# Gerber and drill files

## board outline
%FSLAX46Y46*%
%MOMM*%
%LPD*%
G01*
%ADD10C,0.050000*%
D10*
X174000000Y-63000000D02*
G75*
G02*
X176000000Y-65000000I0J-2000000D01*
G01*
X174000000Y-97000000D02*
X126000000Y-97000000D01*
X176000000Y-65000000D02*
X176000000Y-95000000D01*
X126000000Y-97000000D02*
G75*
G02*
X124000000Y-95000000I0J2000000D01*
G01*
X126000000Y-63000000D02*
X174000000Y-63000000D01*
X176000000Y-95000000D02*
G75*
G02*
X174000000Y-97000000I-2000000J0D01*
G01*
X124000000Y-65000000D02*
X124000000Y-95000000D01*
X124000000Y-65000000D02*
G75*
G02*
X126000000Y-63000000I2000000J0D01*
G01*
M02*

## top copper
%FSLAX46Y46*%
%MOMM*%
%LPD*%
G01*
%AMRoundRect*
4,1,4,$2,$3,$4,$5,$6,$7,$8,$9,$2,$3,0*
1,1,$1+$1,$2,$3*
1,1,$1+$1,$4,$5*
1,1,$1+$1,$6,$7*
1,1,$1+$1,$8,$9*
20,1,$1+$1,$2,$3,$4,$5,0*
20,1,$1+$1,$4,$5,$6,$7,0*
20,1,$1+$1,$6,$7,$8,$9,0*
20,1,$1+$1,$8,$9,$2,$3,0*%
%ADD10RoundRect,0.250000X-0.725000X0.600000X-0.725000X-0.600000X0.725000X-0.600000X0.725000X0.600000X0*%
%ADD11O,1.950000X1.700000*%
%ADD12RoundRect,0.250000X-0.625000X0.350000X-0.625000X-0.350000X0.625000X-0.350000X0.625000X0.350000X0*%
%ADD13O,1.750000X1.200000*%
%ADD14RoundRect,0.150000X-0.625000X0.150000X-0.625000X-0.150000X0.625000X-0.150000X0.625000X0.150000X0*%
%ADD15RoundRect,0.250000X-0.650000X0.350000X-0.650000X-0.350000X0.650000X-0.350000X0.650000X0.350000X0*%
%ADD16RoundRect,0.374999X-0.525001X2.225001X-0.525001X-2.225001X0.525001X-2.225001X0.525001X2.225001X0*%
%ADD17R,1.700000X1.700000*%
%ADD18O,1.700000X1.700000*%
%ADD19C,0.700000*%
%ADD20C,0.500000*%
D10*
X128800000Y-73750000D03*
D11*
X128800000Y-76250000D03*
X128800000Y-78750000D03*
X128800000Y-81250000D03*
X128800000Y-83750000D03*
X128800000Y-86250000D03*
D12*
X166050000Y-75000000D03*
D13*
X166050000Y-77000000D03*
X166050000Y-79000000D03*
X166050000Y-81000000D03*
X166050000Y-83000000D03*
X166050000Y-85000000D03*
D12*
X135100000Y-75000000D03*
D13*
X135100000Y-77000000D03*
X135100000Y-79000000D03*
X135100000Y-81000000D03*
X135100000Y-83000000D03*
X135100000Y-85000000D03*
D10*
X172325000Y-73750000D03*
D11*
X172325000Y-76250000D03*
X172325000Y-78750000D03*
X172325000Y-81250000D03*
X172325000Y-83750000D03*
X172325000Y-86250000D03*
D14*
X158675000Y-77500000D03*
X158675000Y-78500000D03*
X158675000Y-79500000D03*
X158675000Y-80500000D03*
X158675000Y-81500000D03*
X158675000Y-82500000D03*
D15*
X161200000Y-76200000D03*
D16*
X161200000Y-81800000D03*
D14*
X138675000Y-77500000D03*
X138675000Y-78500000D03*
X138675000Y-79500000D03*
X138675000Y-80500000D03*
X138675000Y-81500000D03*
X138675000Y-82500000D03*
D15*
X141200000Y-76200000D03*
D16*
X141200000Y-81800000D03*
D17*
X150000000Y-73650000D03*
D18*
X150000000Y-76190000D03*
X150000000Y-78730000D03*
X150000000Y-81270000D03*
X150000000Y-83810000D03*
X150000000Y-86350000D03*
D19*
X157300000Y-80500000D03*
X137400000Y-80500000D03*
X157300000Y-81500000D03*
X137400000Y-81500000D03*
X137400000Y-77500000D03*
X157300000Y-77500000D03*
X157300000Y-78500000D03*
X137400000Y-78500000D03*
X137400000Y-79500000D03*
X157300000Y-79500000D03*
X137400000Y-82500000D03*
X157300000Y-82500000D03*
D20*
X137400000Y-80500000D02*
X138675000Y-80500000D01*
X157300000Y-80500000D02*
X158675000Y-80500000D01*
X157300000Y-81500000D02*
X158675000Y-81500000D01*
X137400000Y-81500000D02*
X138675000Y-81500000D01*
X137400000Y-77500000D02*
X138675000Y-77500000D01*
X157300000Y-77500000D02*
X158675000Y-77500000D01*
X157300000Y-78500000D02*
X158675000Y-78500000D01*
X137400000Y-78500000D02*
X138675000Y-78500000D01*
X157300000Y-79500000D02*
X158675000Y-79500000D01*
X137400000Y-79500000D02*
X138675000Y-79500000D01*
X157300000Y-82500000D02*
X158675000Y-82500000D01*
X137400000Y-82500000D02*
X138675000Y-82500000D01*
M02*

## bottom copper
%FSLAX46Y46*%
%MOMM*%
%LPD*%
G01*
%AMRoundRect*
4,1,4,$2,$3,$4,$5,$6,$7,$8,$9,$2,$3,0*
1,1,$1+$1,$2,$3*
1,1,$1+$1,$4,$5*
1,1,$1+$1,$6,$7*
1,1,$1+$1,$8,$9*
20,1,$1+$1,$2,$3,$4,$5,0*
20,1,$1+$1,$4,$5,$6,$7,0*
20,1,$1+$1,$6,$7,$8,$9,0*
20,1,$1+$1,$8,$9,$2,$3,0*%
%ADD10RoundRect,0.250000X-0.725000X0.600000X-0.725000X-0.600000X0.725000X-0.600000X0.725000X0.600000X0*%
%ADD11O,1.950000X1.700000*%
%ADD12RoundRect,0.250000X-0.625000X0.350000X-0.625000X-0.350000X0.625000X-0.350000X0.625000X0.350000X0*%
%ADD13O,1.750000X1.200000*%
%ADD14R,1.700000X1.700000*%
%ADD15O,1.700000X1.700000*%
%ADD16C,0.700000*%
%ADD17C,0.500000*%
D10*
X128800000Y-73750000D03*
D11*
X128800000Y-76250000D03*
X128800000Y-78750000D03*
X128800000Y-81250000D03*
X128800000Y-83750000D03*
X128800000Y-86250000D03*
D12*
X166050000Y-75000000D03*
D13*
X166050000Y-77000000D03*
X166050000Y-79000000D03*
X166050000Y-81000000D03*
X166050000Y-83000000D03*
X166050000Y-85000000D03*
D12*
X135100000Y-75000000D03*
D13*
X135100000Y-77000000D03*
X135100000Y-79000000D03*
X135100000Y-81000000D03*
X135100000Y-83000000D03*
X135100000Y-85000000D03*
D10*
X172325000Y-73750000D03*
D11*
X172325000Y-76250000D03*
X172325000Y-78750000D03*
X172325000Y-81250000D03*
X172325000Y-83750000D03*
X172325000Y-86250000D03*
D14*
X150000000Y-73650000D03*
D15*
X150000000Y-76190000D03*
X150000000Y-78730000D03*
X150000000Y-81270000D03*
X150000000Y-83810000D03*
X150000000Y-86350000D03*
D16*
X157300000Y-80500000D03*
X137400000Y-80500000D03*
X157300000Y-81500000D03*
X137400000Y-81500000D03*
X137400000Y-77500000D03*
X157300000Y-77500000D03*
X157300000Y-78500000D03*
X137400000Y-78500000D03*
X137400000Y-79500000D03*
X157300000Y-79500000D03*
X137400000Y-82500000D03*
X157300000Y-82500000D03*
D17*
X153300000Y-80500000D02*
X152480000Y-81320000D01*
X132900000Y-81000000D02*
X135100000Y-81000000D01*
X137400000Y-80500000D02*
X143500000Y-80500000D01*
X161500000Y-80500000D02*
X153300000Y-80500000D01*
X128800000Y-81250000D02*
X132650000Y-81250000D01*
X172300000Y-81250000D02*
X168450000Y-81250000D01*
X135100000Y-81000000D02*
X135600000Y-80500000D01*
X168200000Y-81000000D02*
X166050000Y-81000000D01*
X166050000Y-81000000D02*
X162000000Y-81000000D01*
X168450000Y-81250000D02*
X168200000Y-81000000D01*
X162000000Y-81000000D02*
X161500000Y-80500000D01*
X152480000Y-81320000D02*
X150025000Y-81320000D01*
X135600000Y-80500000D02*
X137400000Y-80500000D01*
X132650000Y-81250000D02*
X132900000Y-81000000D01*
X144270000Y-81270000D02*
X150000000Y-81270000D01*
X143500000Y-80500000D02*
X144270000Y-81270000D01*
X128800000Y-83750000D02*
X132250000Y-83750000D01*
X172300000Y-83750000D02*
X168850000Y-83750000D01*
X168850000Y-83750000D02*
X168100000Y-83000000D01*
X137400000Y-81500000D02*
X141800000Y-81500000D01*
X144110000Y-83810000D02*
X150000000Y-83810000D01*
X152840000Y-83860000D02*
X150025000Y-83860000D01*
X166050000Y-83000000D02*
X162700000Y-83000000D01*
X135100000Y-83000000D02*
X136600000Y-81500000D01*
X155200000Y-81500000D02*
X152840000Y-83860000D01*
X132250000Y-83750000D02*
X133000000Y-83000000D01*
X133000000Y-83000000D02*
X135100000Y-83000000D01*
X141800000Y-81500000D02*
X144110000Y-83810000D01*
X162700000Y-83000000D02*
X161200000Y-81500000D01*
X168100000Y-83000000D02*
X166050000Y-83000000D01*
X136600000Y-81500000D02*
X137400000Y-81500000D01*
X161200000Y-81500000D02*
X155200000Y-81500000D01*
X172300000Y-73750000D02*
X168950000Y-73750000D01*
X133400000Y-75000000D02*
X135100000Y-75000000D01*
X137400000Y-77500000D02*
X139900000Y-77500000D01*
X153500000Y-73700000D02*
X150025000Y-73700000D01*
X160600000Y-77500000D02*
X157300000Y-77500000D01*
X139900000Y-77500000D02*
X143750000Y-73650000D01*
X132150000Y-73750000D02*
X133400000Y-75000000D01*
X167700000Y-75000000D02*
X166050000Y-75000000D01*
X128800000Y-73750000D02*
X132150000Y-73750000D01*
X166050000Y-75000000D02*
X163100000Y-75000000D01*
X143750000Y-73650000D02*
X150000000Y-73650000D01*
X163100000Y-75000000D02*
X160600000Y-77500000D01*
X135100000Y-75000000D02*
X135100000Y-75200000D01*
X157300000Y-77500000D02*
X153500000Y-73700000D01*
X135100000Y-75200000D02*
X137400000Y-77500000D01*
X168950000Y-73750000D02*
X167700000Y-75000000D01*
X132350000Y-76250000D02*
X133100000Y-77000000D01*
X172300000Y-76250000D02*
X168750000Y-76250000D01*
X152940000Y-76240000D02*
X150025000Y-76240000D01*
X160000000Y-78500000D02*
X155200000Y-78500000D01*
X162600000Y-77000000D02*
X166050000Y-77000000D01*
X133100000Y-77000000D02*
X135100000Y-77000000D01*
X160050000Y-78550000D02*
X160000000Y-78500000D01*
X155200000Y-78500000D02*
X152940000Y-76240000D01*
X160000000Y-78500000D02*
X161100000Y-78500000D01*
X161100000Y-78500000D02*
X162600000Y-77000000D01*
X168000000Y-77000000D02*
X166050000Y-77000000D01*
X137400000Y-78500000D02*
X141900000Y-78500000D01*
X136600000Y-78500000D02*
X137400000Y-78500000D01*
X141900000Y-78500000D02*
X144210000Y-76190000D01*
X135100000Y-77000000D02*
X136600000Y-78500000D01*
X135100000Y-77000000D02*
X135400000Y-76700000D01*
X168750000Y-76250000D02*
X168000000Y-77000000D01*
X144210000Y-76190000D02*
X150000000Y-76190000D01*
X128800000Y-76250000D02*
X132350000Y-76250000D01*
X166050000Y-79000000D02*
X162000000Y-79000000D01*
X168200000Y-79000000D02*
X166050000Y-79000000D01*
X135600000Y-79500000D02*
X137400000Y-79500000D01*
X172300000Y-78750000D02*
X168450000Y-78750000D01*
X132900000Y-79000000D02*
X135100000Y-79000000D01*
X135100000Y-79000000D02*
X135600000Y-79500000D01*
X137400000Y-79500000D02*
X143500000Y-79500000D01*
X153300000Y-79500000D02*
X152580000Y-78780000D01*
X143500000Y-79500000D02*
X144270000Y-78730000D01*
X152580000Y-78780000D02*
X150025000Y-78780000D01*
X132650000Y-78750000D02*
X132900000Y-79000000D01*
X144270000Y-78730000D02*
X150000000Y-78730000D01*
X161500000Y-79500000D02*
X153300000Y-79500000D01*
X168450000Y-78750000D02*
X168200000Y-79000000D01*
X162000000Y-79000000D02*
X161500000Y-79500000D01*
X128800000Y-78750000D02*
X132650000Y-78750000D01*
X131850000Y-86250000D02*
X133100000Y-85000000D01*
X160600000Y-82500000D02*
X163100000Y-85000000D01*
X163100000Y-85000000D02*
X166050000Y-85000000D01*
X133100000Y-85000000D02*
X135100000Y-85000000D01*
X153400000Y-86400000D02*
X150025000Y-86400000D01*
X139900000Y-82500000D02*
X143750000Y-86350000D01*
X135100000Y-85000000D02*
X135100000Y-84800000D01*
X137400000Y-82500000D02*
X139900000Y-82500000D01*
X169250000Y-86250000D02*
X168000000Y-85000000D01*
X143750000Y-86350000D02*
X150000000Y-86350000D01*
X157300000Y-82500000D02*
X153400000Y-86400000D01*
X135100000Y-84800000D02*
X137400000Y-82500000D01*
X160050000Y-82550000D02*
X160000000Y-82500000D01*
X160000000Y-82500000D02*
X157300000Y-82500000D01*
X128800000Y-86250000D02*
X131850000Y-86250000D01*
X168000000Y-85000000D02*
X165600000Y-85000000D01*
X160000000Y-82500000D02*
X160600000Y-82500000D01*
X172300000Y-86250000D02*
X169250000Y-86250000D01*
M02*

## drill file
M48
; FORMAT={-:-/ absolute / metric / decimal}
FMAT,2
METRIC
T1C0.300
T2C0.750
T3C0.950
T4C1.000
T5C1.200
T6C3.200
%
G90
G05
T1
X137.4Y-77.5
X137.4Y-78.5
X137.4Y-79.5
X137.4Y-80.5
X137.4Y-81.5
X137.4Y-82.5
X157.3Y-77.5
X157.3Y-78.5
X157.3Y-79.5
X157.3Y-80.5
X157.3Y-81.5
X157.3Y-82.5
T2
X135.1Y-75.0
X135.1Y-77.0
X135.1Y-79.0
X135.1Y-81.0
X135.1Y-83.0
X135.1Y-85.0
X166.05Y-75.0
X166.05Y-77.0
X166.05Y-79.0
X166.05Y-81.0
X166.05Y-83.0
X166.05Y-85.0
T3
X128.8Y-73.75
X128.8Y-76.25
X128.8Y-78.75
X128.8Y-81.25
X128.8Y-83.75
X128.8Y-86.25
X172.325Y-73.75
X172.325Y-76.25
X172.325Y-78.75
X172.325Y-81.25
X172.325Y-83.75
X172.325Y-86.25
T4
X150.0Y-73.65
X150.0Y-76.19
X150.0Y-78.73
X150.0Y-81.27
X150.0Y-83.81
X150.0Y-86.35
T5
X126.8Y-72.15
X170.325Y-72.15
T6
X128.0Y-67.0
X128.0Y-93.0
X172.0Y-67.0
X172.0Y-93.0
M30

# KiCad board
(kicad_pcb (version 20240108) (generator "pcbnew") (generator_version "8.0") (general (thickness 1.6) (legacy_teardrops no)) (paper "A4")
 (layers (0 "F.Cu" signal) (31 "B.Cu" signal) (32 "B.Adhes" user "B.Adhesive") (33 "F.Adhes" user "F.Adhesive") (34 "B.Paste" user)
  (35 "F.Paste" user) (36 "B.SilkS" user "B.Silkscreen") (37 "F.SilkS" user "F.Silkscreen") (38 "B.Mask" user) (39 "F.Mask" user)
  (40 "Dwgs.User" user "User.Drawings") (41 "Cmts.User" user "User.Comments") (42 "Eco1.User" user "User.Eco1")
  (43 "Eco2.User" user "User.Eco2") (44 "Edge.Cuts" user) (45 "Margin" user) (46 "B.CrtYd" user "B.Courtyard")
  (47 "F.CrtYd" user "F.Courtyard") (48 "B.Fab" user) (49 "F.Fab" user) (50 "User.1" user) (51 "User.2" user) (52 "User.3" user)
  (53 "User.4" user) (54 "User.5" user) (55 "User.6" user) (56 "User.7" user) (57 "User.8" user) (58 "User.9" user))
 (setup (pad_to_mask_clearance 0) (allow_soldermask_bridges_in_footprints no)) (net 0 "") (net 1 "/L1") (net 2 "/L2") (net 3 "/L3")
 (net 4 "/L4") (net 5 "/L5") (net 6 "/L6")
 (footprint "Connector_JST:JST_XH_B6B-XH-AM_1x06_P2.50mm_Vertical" (layer "F.Cu") (at 128.8 73.75 -90)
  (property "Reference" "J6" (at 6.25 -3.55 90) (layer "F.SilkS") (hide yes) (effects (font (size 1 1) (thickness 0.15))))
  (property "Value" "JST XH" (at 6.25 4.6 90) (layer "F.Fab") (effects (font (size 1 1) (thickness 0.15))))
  (pad "" np_thru_hole circle (at -1.6 2 270) (size 1.2 1.2) (drill 1.2) (layers "*.Cu" "*.Mask"))
  (pad "1" thru_hole roundrect (at 0 0 270) (size 1.7 1.95) (drill 0.95) (layers "*.Cu" "*.Mask") (remove_unused_layers no)
   (roundrect_rratio 0.1470588235) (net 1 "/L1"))
  (pad "2" thru_hole oval (at 2.5 0 270) (size 1.7 1.95) (drill 0.95) (layers "*.Cu" "*.Mask") (remove_unused_layers no) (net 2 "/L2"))
  (pad "3" thru_hole oval (at 5 0 270) (size 1.7 1.95) (drill 0.95) (layers "*.Cu" "*.Mask") (remove_unused_layers no) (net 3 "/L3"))
  (pad "4" thru_hole oval (at 7.5 0 270) (size 1.7 1.95) (drill 0.95) (layers "*.Cu" "*.Mask") (remove_unused_layers no) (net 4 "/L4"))
  (pad "5" thru_hole oval (at 10 0 270) (size 1.7 1.95) (drill 0.95) (layers "*.Cu" "*.Mask") (remove_unused_layers no) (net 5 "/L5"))
  (pad "6" thru_hole oval (at 12.5 0 270) (size 1.7 1.95) (drill 0.95) (layers "*.Cu" "*.Mask") (remove_unused_layers no) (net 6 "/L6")))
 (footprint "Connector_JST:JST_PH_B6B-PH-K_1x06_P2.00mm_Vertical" (layer "F.Cu") (at 166.05 75 -90)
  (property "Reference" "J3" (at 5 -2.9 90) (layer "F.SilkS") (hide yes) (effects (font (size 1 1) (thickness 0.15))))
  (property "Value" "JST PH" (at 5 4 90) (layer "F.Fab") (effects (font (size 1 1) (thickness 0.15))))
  (pad "1" thru_hole roundrect (at 0 0 270) (size 1.2 1.75) (drill 0.75) (layers "*.Cu" "*.Mask") (remove_unused_layers no)
   (roundrect_rratio 0.2083333333) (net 1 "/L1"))
  (pad "2" thru_hole oval (at 2 0 270) (size 1.2 1.75) (drill 0.75) (layers "*.Cu" "*.Mask") (remove_unused_layers no) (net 2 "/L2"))
  (pad "3" thru_hole oval (at 4 0 270) (size 1.2 1.75) (drill 0.75) (layers "*.Cu" "*.Mask") (remove_unused_layers no) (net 3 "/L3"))
  (pad "4" thru_hole oval (at 6 0 270) (size 1.2 1.75) (drill 0.75) (layers "*.Cu" "*.Mask") (remove_unused_layers no) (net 4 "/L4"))
  (pad "5" thru_hole oval (at 8 0 270) (size 1.2 1.75) (drill 0.75) (layers "*.Cu" "*.Mask") (remove_unused_layers no) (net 5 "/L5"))
  (pad "6" thru_hole oval (at 10 0 270) (size 1.2 1.75) (drill 0.75) (layers "*.Cu" "*.Mask") (remove_unused_layers no) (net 6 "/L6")))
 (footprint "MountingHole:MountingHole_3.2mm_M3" (layer "F.Cu") (at 172 93)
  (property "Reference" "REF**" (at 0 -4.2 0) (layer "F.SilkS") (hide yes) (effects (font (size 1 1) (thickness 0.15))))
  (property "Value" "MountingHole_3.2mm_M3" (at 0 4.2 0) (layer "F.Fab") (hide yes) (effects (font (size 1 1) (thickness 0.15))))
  (pad "" np_thru_hole circle (at 0 0) (size 3.2 3.2) (drill 3.2) (layers "F&B.Cu" "*.Mask")))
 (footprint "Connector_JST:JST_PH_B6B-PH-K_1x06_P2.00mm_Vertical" (layer "F.Cu") (at 135.1 75 -90)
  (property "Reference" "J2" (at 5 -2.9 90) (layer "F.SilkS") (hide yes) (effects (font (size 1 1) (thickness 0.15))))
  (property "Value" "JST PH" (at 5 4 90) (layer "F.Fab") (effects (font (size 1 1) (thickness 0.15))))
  (pad "1" thru_hole roundrect (at 0 0 270) (size 1.2 1.75) (drill 0.75) (layers "*.Cu" "*.Mask") (remove_unused_layers no)
   (roundrect_rratio 0.2083333333) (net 1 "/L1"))
  (pad "2" thru_hole oval (at 2 0 270) (size 1.2 1.75) (drill 0.75) (layers "*.Cu" "*.Mask") (remove_unused_layers no) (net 2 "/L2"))
  (pad "3" thru_hole oval (at 4 0 270) (size 1.2 1.75) (drill 0.75) (layers "*.Cu" "*.Mask") (remove_unused_layers no) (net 3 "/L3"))
  (pad "4" thru_hole oval (at 6 0 270) (size 1.2 1.75) (drill 0.75) (layers "*.Cu" "*.Mask") (remove_unused_layers no) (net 4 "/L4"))
  (pad "5" thru_hole oval (at 8 0 270) (size 1.2 1.75) (drill 0.75) (layers "*.Cu" "*.Mask") (remove_unused_layers no) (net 5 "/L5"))
  (pad "6" thru_hole oval (at 10 0 270) (size 1.2 1.75) (drill 0.75) (layers "*.Cu" "*.Mask") (remove_unused_layers no) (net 6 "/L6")))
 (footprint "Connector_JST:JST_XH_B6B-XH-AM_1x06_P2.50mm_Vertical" (layer "F.Cu") (at 172.325 73.75 -90)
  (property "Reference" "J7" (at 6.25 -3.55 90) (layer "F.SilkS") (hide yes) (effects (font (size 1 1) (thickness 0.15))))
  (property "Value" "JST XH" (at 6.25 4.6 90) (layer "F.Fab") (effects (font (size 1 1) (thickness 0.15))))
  (pad "" np_thru_hole circle (at -1.6 2 270) (size 1.2 1.2) (drill 1.2) (layers "*.Cu" "*.Mask"))
  (pad "1" thru_hole roundrect (at 0 0 270) (size 1.7 1.95) (drill 0.95) (layers "*.Cu" "*.Mask") (remove_unused_layers no)
   (roundrect_rratio 0.1470588235) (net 1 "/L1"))
  (pad "2" thru_hole oval (at 2.5 0 270) (size 1.7 1.95) (drill 0.95) (layers "*.Cu" "*.Mask") (remove_unused_layers no) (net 2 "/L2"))
  (pad "3" thru_hole oval (at 5 0 270) (size 1.7 1.95) (drill 0.95) (layers "*.Cu" "*.Mask") (remove_unused_layers no) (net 3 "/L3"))
  (pad "4" thru_hole oval (at 7.5 0 270) (size 1.7 1.95) (drill 0.95) (layers "*.Cu" "*.Mask") (remove_unused_layers no) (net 4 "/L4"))
  (pad "5" thru_hole oval (at 10 0 270) (size 1.7 1.95) (drill 0.95) (layers "*.Cu" "*.Mask") (remove_unused_layers no) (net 5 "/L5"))
  (pad "6" thru_hole oval (at 12.5 0 270) (size 1.7 1.95) (drill 0.95) (layers "*.Cu" "*.Mask") (remove_unused_layers no) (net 6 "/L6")))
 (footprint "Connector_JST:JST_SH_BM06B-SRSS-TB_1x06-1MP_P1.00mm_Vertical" (layer "F.Cu") (at 160 80 -90)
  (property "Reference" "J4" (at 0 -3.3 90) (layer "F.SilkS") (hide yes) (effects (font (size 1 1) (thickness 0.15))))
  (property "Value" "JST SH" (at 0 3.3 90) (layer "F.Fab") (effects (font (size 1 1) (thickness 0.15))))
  (pad "1" smd roundrect (at -2.5 1.325 270) (size 0.6 1.55) (layers "F.Cu" "F.Paste" "F.Mask") (roundrect_rratio 0.25) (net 1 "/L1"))
  (pad "2" smd roundrect (at -1.5 1.325 270) (size 0.6 1.55) (layers "F.Cu" "F.Paste" "F.Mask") (roundrect_rratio 0.25) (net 2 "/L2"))
  (pad "3" smd roundrect (at -0.5 1.325 270) (size 0.6 1.55) (layers "F.Cu" "F.Paste" "F.Mask") (roundrect_rratio 0.25) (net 3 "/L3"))
  (pad "4" smd roundrect (at 0.5 1.325 270) (size 0.6 1.55) (layers "F.Cu" "F.Paste" "F.Mask") (roundrect_rratio 0.25) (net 4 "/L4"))
  (pad "5" smd roundrect (at 1.5 1.325 270) (size 0.6 1.55) (layers "F.Cu" "F.Paste" "F.Mask") (roundrect_rratio 0.25) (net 5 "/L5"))
  (pad "6" smd roundrect (at 2.5 1.325 270) (size 0.6 1.55) (layers "F.Cu" "F.Paste" "F.Mask") (roundrect_rratio 0.25) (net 6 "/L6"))
  (pad "MP" smd roundrect (at -3.8 -1.2 270) (size 1.2 1.8) (layers "F.Cu" "F.Paste" "F.Mask") (roundrect_rratio 0.2083333333))
  (pad "MP" smd roundrect (at 1.8 -1.2 270) (size 5.2 1.8) (layers "F.Cu" "F.Paste" "F.Mask") (roundrect_rratio 0.2083327778)))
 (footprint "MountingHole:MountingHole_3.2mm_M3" (layer "F.Cu") (at 172 67)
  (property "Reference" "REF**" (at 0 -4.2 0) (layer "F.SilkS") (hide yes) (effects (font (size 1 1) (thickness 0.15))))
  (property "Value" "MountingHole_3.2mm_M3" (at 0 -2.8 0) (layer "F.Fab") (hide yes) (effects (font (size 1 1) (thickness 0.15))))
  (pad "" np_thru_hole circle (at 0 0) (size 3.2 3.2) (drill 3.2) (layers "F&B.Cu" "*.Mask")))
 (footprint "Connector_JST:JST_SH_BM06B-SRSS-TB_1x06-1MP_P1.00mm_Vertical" (layer "F.Cu") (at 140 80 -90)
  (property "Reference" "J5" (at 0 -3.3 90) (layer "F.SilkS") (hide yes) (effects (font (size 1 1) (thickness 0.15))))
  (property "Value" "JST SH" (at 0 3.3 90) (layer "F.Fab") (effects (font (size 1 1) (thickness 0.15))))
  (pad "1" smd roundrect (at -2.5 1.325 270) (size 0.6 1.55) (layers "F.Cu" "F.Paste" "F.Mask") (roundrect_rratio 0.25) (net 1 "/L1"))
  (pad "2" smd roundrect (at -1.5 1.325 270) (size 0.6 1.55) (layers "F.Cu" "F.Paste" "F.Mask") (roundrect_rratio 0.25) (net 2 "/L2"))
  (pad "3" smd roundrect (at -0.5 1.325 270) (size 0.6 1.55) (layers "F.Cu" "F.Paste" "F.Mask") (roundrect_rratio 0.25) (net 3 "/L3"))
  (pad "4" smd roundrect (at 0.5 1.325 270) (size 0.6 1.55) (layers "F.Cu" "F.Paste" "F.Mask") (roundrect_rratio 0.25) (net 4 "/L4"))
  (pad "5" smd roundrect (at 1.5 1.325 270) (size 0.6 1.55) (layers "F.Cu" "F.Paste" "F.Mask") (roundrect_rratio 0.25) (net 5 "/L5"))
  (pad "6" smd roundrect (at 2.5 1.325 270) (size 0.6 1.55) (layers "F.Cu" "F.Paste" "F.Mask") (roundrect_rratio 0.25) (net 6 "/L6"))
  (pad "MP" smd roundrect (at -3.8 -1.2 270) (size 1.2 1.8) (layers "F.Cu" "F.Paste" "F.Mask") (roundrect_rratio 0.2083333333))
  (pad "MP" smd roundrect (at 1.8 -1.2 270) (size 5.2 1.8) (layers "F.Cu" "F.Paste" "F.Mask") (roundrect_rratio 0.2083327778)))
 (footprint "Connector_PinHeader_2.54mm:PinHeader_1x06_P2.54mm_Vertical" (layer "F.Cu") (at 150 80)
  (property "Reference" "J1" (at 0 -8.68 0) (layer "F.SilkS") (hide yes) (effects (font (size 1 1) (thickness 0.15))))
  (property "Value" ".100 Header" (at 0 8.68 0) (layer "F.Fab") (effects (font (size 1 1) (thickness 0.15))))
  (pad "1" thru_hole rect (at 0 -6.35) (size 1.7 1.7) (drill 1) (layers "*.Cu" "*.Mask") (remove_unused_layers no) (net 1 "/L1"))
  (pad "2" thru_hole oval (at 0 -3.81) (size 1.7 1.7) (drill 1) (layers "*.Cu" "*.Mask") (remove_unused_layers no) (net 2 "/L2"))
  (pad "3" thru_hole oval (at 0 -1.27) (size 1.7 1.7) (drill 1) (layers "*.Cu" "*.Mask") (remove_unused_layers no) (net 3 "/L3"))
  (pad "4" thru_hole oval (at 0 1.27) (size 1.7 1.7) (drill 1) (layers "*.Cu" "*.Mask") (remove_unused_layers no) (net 4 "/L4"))
  (pad "5" thru_hole oval (at 0 3.81) (size 1.7 1.7) (drill 1) (layers "*.Cu" "*.Mask") (remove_unused_layers no) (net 5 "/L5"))
  (pad "6" thru_hole oval (at 0 6.35) (size 1.7 1.7) (drill 1) (layers "*.Cu" "*.Mask") (remove_unused_layers no) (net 6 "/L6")))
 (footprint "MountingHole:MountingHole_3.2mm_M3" (layer "F.Cu") (at 128 93)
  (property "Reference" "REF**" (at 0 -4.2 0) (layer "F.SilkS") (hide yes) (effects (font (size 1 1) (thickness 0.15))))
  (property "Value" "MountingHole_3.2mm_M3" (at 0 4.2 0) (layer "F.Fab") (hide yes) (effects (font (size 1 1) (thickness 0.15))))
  (pad "" np_thru_hole circle (at 0 0) (size 3.2 3.2) (drill 3.2) (layers "F&B.Cu" "*.Mask")))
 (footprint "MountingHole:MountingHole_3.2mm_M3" (layer "F.Cu") (at 128 67)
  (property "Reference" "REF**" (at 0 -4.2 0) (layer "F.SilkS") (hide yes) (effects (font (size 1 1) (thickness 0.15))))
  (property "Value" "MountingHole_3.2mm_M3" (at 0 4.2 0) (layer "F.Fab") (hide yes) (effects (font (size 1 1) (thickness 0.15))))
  (pad "" np_thru_hole circle (at 0 0) (size 3.2 3.2) (drill 3.2) (layers "*.Cu" "*.Mask")))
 (gr_arc (start 174 63) (mid 175.414214 63.585786) (end 176 65) (stroke (width 0.05) (type default)) (layer "Edge.Cuts"))
 (gr_line (start 174 97) (end 126 97) (stroke (width 0.05) (type default)) (layer "Edge.Cuts"))
 (gr_line (start 176 65) (end 176 95) (stroke (width 0.05) (type default)) (layer "Edge.Cuts"))
 (gr_arc (start 126 97) (mid 124.585786 96.414214) (end 124 95) (stroke (width 0.05) (type default)) (layer "Edge.Cuts"))
 (gr_line (start 126 63) (end 174 63) (stroke (width 0.05) (type default)) (layer "Edge.Cuts"))
 (gr_arc (start 176 95) (mid 175.414214 96.414214) (end 174 97) (stroke (width 0.05) (type default)) (layer "Edge.Cuts"))
 (gr_line (start 124 65) (end 124 95) (stroke (width 0.05) (type default)) (layer "Edge.Cuts"))
 (gr_arc (start 124 65) (mid 124.585786 63.585786) (end 126 63) (stroke (width 0.05) (type default)) (layer "Edge.Cuts"))
 (segment (start 137.4 80.5) (end 138.675 80.5) (width 0.5) (layer "F.Cu") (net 4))
 (segment (start 157.3 80.5) (end 158.675 80.5) (width 0.5) (layer "F.Cu") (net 4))
 (via (at 157.3 80.5) (size 0.7) (drill 0.3) (layers "F.Cu" "B.Cu") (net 4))
 (via (at 137.4 80.5) (size 0.7) (drill 0.3) (layers "F.Cu" "B.Cu") (free yes) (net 4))
 (segment (start 153.3 80.5) (end 152.48 81.32) (width 0.5) (layer "B.Cu") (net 4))
 (segment (start 132.9 81) (end 135.1 81) (width 0.5) (layer "B.Cu") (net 4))
 (segment (start 137.4 80.5) (end 143.5 80.5) (width 0.5) (layer "B.Cu") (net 4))
 (segment (start 161.5 80.5) (end 153.3 80.5) (width 0.5) (layer "B.Cu") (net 4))
 (segment (start 128.8 81.25) (end 132.65 81.25) (width 0.5) (layer "B.Cu") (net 4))
 (segment (start 172.3 81.25) (end 168.45 81.25) (width 0.5) (layer "B.Cu") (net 4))
 (segment (start 135.1 81) (end 135.6 80.5) (width 0.5) (layer "B.Cu") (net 4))
 (segment (start 168.2 81) (end 166.05 81) (width 0.5) (layer "B.Cu") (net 4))
 (segment (start 166.05 81) (end 162 81) (width 0.5) (layer "B.Cu") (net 4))
 (segment (start 168.45 81.25) (end 168.2 81) (width 0.5) (layer "B.Cu") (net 4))
 (segment (start 162 81) (end 161.5 80.5) (width 0.5) (layer "B.Cu") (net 4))
 (segment (start 152.48 81.32) (end 150.025 81.32) (width 0.5) (layer "B.Cu") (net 4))
 (segment (start 135.6 80.5) (end 137.4 80.5) (width 0.5) (layer "B.Cu") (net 4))
 (segment (start 132.65 81.25) (end 132.9 81) (width 0.5) (layer "B.Cu") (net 4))
 (segment (start 144.27 81.27) (end 150 81.27) (width 0.5) (layer "B.Cu") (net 4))
 (segment (start 143.5 80.5) (end 144.27 81.27) (width 0.5) (layer "B.Cu") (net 4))
 (segment (start 157.3 81.5) (end 158.675 81.5) (width 0.5) (layer "F.Cu") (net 5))
 (segment (start 137.4 81.5) (end 138.675 81.5) (width 0.5) (layer "F.Cu") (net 5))
 (via (at 157.3 81.5) (size 0.7) (drill 0.3) (layers "F.Cu" "B.Cu") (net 5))
 (via (at 137.4 81.5) (size 0.7) (drill 0.3) (layers "F.Cu" "B.Cu") (free yes) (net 5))
 (segment (start 128.8 83.75) (end 132.25 83.75) (width 0.5) (layer "B.Cu") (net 5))
 (segment (start 172.3 83.75) (end 168.85 83.75) (width 0.5) (layer "B.Cu") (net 5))
 (segment (start 168.85 83.75) (end 168.1 83) (width 0.5) (layer "B.Cu") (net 5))
 (segment (start 137.4 81.5) (end 141.8 81.5) (width 0.5) (layer "B.Cu") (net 5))
 (segment (start 144.11 83.81) (end 150 83.81) (width 0.5) (layer "B.Cu") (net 5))
 (segment (start 152.84 83.86) (end 150.025 83.86) (width 0.5) (layer "B.Cu") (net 5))
 (segment (start 166.05 83) (end 162.7 83) (width 0.5) (layer "B.Cu") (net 5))
 (segment (start 135.1 83) (end 136.6 81.5) (width 0.5) (layer "B.Cu") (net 5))
 (segment (start 155.2 81.5) (end 152.84 83.86) (width 0.5) (layer "B.Cu") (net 5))
 (segment (start 132.25 83.75) (end 133 83) (width 0.5) (layer "B.Cu") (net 5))
 (segment (start 133 83) (end 135.1 83) (width 0.5) (layer "B.Cu") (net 5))
 (segment (start 141.8 81.5) (end 144.11 83.81) (width 0.5) (layer "B.Cu") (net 5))
 (segment (start 162.7 83) (end 161.2 81.5) (width 0.5) (layer "B.Cu") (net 5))
 (segment (start 168.1 83) (end 166.05 83) (width 0.5) (layer "B.Cu") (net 5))
 (segment (start 136.6 81.5) (end 137.4 81.5) (width 0.5) (layer "B.Cu") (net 5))
 (segment (start 161.2 81.5) (end 155.2 81.5) (width 0.5) (layer "B.Cu") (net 5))
 (segment (start 137.4 77.5) (end 138.675 77.5) (width 0.5) (layer "F.Cu") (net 1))
 (segment (start 157.3 77.5) (end 158.675 77.5) (width 0.5) (layer "F.Cu") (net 1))
 (via (at 137.4 77.5) (size 0.7) (drill 0.3) (layers "F.Cu" "B.Cu") (free yes) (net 1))
 (via (at 157.3 77.5) (size 0.7) (drill 0.3) (layers "F.Cu" "B.Cu") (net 1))
 (segment (start 172.3 73.75) (end 168.95 73.75) (width 0.5) (layer "B.Cu") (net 1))
 (segment (start 133.4 75) (end 135.1 75) (width 0.5) (layer "B.Cu") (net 1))
 (segment (start 137.4 77.5) (end 139.9 77.5) (width 0.5) (layer "B.Cu") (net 1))
 (segment (start 153.5 73.7) (end 150.025 73.7) (width 0.5) (layer "B.Cu") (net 1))
 (segment (start 160.6 77.5) (end 157.3 77.5) (width 0.5) (layer "B.Cu") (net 1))
 (segment (start 139.9 77.5) (end 143.75 73.65) (width 0.5) (layer "B.Cu") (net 1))
 (segment (start 132.15 73.75) (end 133.4 75) (width 0.5) (layer "B.Cu") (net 1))
 (segment (start 167.7 75) (end 166.05 75) (width 0.5) (layer "B.Cu") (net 1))
 (segment (start 128.8 73.75) (end 132.15 73.75) (width 0.5) (layer "B.Cu") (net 1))
 (segment (start 166.05 75) (end 163.1 75) (width 0.5) (layer "B.Cu") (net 1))
 (segment (start 143.75 73.65) (end 150 73.65) (width 0.5) (layer "B.Cu") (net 1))
 (segment (start 163.1 75) (end 160.6 77.5) (width 0.5) (layer "B.Cu") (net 1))
 (segment (start 135.1 75) (end 135.1 75.2) (width 0.5) (layer "B.Cu") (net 1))
 (segment (start 157.3 77.5) (end 153.5 73.7) (width 0.5) (layer "B.Cu") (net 1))
 (segment (start 135.1 75.2) (end 137.4 77.5) (width 0.5) (layer "B.Cu") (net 1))
 (segment (start 168.95 73.75) (end 167.7 75) (width 0.5) (layer "B.Cu") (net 1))
 (segment (start 157.3 78.5) (end 158.675 78.5) (width 0.5) (layer "F.Cu") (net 2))
 (segment (start 137.4 78.5) (end 138.675 78.5) (width 0.5) (layer "F.Cu") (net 2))
 (via (at 157.3 78.5) (size 0.7) (drill 0.3) (layers "F.Cu" "B.Cu") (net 2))
 (via (at 137.4 78.5) (size 0.7) (drill 0.3) (layers "F.Cu" "B.Cu") (free yes) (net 2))
 (segment (start 132.35 76.25) (end 133.1 77) (width 0.5) (layer "B.Cu") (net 2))
 (segment (start 172.3 76.25) (end 168.75 76.25) (width 0.5) (layer "B.Cu") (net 2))
 (segment (start 152.94 76.24) (end 150.025 76.24) (width 0.5) (layer "B.Cu") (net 2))
 (segment (start 160 78.5) (end 155.2 78.5) (width 0.5) (layer "B.Cu") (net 2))
 (segment (start 162.6 77) (end 166.05 77) (width 0.5) (layer "B.Cu") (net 2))
 (segment (start 133.1 77) (end 135.1 77) (width 0.5) (layer "B.Cu") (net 2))
 (segment (start 160.05 78.55) (end 160 78.5) (width 0.5) (layer "B.Cu") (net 2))
 (segment (start 155.2 78.5) (end 152.94 76.24) (width 0.5) (layer "B.Cu") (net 2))
 (segment (start 160 78.5) (end 161.1 78.5) (width 0.5) (layer "B.Cu") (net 2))
 (segment (start 161.1 78.5) (end 162.6 77) (width 0.5) (layer "B.Cu") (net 2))
 (segment (start 168 77) (end 166.05 77) (width 0.5) (layer "B.Cu") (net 2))
 (segment (start 137.4 78.5) (end 141.9 78.5) (width 0.5) (layer "B.Cu") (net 2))
 (segment (start 136.6 78.5) (end 137.4 78.5) (width 0.5) (layer "B.Cu") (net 2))
 (segment (start 141.9 78.5) (end 144.21 76.19) (width 0.5) (layer "B.Cu") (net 2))
 (segment (start 135.1 77) (end 136.6 78.5) (width 0.5) (layer "B.Cu") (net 2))
 (segment (start 135.1 77) (end 135.4 76.7) (width 0.5) (layer "B.Cu") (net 2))
 (segment (start 168.75 76.25) (end 168 77) (width 0.5) (layer "B.Cu") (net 2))
 (segment (start 144.21 76.19) (end 150 76.19) (width 0.5) (layer "B.Cu") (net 2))
 (segment (start 128.8 76.25) (end 132.35 76.25) (width 0.5) (layer "B.Cu") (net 2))
 (segment (start 157.3 79.5) (end 158.675 79.5) (width 0.5) (layer "F.Cu") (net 3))
 (segment (start 137.4 79.5) (end 138.675 79.5) (width 0.5) (layer "F.Cu") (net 3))
 (via (at 137.4 79.5) (size 0.7) (drill 0.3) (layers "F.Cu" "B.Cu") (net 3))
 (via (at 157.3 79.5) (size 0.7) (drill 0.3) (layers "F.Cu" "B.Cu") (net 3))
 (segment (start 166.05 79) (end 162 79) (width 0.5) (layer "B.Cu") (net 3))
 (segment (start 168.2 79) (end 166.05 79) (width 0.5) (layer "B.Cu") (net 3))
 (segment (start 135.6 79.5) (end 137.4 79.5) (width 0.5) (layer "B.Cu") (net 3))
 (segment (start 172.3 78.75) (end 168.45 78.75) (width 0.5) (layer "B.Cu") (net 3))
 (segment (start 132.9 79) (end 135.1 79) (width 0.5) (layer "B.Cu") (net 3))
 (segment (start 135.1 79) (end 135.6 79.5) (width 0.5) (layer "B.Cu") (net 3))
 (segment (start 137.4 79.5) (end 143.5 79.5) (width 0.5) (layer "B.Cu") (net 3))
 (segment (start 153.3 79.5) (end 152.58 78.78) (width 0.5) (layer "B.Cu") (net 3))
 (segment (start 143.5 79.5) (end 144.27 78.73) (width 0.5) (layer "B.Cu") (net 3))
 (segment (start 152.58 78.78) (end 150.025 78.78) (width 0.5) (layer "B.Cu") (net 3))
 (segment (start 132.65 78.75) (end 132.9 79) (width 0.5) (layer "B.Cu") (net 3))
 (segment (start 144.27 78.73) (end 150 78.73) (width 0.5) (layer "B.Cu") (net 3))
 (segment (start 161.5 79.5) (end 153.3 79.5) (width 0.5) (layer "B.Cu") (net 3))
 (segment (start 168.45 78.75) (end 168.2 79) (width 0.5) (layer "B.Cu") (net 3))
 (segment (start 162 79) (end 161.5 79.5) (width 0.5) (layer "B.Cu") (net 3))
 (segment (start 128.8 78.75) (end 132.65 78.75) (width 0.5) (layer "B.Cu") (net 3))
 (segment (start 157.3 82.5) (end 158.675 82.5) (width 0.5) (layer "F.Cu") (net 6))
 (segment (start 137.4 82.5) (end 138.675 82.5) (width 0.5) (layer "F.Cu") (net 6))
 (via (at 137.4 82.5) (size 0.7) (drill 0.3) (layers "F.Cu" "B.Cu") (free yes) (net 6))
 (via (at 157.3 82.5) (size 0.7) (drill 0.3) (layers "F.Cu" "B.Cu") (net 6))
 (segment (start 131.85 86.25) (end 133.1 85) (width 0.5) (layer "B.Cu") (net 6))
 (segment (start 160.6 82.5) (end 163.1 85) (width 0.5) (layer "B.Cu") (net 6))
 (segment (start 163.1 85) (end 166.05 85) (width 0.5) (layer "B.Cu") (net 6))
 (segment (start 133.1 85) (end 135.1 85) (width 0.5) (layer "B.Cu") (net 6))
 (segment (start 153.4 86.4) (end 150.025 86.4) (width 0.5) (layer "B.Cu") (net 6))
 (segment (start 139.9 82.5) (end 143.75 86.35) (width 0.5) (layer "B.Cu") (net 6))
 (segment (start 135.1 85) (end 135.1 84.8) (width 0.5) (layer "B.Cu") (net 6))
 (segment (start 137.4 82.5) (end 139.9 82.5) (width 0.5) (layer "B.Cu") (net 6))
 (segment (start 169.25 86.25) (end 168 85) (width 0.5) (layer "B.Cu") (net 6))
 (segment (start 143.75 86.35) (end 150 86.35) (width 0.5) (layer "B.Cu") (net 6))
 (segment (start 157.3 82.5) (end 153.4 86.4) (width 0.5) (layer "B.Cu") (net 6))
 (segment (start 135.1 84.8) (end 137.4 82.5) (width 0.5) (layer "B.Cu") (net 6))
 (segment (start 160.05 82.55) (end 160 82.5) (width 0.5) (layer "B.Cu") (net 6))
 (segment (start 160 82.5) (end 157.3 82.5) (width 0.5) (layer "B.Cu") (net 6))
 (segment (start 128.8 86.25) (end 131.85 86.25) (width 0.5) (layer "B.Cu") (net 6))
 (segment (start 168 85) (end 165.6 85) (width 0.5) (layer "B.Cu") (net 6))
 (segment (start 160 82.5) (end 160.6 82.5) (width 0.5) (layer "B.Cu") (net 6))
 (segment (start 172.3 86.25) (end 169.25 86.25) (width 0.5) (layer "B.Cu") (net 6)))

